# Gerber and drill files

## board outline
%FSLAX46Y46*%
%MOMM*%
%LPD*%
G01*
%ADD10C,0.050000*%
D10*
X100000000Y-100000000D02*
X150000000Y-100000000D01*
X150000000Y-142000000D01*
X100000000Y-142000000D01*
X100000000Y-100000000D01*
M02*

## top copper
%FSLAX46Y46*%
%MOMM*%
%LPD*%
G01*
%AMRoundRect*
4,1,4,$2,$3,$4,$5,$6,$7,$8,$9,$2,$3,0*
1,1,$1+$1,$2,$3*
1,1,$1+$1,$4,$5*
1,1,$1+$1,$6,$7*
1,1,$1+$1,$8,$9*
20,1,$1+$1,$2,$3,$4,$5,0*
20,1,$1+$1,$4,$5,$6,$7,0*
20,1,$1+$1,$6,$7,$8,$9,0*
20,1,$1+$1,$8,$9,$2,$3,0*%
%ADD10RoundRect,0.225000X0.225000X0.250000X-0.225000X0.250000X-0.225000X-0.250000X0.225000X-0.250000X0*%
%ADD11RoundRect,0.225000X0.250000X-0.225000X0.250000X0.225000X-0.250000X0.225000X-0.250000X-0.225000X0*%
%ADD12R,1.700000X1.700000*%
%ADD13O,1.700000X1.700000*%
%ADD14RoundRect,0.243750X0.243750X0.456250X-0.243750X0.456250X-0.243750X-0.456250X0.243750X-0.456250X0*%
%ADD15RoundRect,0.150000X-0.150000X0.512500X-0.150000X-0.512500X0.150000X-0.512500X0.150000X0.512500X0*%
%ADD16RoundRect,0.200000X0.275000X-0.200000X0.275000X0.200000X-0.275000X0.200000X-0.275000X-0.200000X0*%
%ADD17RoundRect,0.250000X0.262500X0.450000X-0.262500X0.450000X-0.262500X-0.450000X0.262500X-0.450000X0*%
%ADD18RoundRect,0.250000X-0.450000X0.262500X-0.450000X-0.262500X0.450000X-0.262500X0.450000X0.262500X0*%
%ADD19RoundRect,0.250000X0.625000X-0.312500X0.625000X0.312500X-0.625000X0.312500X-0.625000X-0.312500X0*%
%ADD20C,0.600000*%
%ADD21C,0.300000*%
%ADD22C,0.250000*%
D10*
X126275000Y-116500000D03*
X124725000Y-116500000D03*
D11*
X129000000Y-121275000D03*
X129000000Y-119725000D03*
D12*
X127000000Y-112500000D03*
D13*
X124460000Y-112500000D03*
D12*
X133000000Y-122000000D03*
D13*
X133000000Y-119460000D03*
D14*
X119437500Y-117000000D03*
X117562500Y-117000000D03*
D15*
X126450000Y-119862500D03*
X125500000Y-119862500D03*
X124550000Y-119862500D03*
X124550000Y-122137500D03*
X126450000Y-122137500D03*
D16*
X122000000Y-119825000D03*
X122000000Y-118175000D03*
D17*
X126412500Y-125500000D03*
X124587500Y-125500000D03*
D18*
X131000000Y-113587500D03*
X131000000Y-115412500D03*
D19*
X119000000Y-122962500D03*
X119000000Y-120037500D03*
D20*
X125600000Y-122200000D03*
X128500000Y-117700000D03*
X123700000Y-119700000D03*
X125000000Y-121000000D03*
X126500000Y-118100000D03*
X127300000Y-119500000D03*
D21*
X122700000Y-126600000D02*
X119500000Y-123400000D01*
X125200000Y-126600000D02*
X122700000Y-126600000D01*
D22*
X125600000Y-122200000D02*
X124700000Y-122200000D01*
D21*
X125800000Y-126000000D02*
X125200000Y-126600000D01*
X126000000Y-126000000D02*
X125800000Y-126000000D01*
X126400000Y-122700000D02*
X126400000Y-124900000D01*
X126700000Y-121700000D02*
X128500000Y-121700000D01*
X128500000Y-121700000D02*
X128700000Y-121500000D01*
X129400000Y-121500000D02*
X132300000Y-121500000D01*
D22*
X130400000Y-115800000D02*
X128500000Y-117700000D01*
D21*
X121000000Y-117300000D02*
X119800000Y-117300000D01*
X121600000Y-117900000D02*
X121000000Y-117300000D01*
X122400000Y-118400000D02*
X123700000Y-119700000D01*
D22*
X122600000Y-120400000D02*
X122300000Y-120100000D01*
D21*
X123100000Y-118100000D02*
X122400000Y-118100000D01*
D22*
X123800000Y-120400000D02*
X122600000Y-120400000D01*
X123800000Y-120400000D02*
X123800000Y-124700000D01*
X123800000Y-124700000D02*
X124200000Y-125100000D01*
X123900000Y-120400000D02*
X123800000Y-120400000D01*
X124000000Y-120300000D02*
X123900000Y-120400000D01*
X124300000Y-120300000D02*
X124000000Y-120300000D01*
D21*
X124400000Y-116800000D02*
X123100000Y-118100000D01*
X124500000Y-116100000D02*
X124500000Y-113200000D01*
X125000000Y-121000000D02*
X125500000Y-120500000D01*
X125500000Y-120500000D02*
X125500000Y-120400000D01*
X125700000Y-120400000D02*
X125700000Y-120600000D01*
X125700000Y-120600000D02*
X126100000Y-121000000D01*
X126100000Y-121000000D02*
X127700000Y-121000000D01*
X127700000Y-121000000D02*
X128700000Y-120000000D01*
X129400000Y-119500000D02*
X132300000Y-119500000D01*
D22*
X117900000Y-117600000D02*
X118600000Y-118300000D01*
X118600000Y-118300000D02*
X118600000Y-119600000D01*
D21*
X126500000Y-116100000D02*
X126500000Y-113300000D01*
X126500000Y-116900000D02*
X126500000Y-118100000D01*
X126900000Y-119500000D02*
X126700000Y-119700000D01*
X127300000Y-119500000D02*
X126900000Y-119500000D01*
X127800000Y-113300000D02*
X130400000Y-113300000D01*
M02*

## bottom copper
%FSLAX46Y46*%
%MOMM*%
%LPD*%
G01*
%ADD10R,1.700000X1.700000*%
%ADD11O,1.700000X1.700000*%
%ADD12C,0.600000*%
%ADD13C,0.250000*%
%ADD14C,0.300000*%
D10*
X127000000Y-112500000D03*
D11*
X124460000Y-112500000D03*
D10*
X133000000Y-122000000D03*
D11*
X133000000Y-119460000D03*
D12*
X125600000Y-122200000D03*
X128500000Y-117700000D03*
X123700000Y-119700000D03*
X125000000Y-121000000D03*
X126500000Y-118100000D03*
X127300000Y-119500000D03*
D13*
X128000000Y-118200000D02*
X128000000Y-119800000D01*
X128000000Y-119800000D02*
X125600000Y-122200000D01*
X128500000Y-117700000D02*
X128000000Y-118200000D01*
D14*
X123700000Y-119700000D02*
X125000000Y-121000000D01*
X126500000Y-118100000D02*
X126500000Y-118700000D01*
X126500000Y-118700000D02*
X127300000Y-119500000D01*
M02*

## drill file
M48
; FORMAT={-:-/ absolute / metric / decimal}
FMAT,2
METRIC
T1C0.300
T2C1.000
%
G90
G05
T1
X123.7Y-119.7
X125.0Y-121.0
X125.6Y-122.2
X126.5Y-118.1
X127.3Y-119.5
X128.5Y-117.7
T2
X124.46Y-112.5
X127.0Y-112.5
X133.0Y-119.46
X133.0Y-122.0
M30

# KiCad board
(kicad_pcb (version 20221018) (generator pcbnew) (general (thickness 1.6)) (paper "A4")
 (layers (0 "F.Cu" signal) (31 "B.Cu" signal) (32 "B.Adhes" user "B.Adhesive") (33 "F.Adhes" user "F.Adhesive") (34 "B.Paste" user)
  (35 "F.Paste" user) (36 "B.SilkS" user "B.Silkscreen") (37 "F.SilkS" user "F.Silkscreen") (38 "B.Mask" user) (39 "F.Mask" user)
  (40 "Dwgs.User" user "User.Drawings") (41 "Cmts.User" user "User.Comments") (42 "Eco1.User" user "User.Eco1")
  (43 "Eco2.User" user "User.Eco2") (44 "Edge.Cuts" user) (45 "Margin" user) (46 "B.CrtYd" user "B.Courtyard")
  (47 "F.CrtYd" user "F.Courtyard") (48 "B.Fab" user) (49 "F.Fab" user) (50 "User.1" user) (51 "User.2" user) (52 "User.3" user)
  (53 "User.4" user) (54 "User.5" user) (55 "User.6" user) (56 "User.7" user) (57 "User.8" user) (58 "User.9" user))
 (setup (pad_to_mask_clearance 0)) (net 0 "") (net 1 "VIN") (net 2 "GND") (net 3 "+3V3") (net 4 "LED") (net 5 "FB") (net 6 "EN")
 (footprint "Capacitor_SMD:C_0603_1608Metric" (layer "F.Cu") (at 125.5 116.5 180)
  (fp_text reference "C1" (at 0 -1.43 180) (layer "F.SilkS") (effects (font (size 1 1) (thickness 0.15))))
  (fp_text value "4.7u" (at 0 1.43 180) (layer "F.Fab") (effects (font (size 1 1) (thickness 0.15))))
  (pad "1" smd roundrect (at -0.775 0 180) (size 0.9 0.95) (layers "F.Cu" "F.Paste" "F.Mask") (roundrect_rratio 0.25) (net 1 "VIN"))
  (pad "2" smd roundrect (at 0.775 0 180) (size 0.9 0.95) (layers "F.Cu" "F.Paste" "F.Mask") (roundrect_rratio 0.25) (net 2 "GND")))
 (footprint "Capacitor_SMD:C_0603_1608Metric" (layer "F.Cu") (at 129 120.5 90)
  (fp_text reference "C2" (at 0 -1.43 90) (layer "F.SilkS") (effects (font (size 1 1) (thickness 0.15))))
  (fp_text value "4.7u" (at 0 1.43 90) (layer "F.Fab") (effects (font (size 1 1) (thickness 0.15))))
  (pad "1" smd roundrect (at -0.775 0 90) (size 0.9 0.95) (layers "F.Cu" "F.Paste" "F.Mask") (roundrect_rratio 0.25) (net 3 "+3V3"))
  (pad "2" smd roundrect (at 0.775 0 90) (size 0.9 0.95) (layers "F.Cu" "F.Paste" "F.Mask") (roundrect_rratio 0.25) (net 2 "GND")))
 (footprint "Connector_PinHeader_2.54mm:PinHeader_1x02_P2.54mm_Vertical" (layer "F.Cu") (at 127 112.5 -90)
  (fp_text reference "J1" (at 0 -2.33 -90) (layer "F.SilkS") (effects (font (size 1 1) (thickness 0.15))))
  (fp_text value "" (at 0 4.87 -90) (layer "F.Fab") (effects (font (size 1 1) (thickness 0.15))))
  (pad "1" thru_hole rect (at 0 0 270) (size 1.7 1.7) (drill 1) (layers "*.Cu" "*.Mask") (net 1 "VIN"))
  (pad "2" thru_hole oval (at 0 2.54 270) (size 1.7 1.7) (drill 1) (layers "*.Cu" "*.Mask") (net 2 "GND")))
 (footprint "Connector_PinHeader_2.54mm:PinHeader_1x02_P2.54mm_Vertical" (layer "F.Cu") (at 133 122 180)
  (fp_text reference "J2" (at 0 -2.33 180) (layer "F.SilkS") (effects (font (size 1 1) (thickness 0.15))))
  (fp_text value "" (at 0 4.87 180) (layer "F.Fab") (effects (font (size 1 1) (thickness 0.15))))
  (pad "1" thru_hole rect (at 0 0 180) (size 1.7 1.7) (drill 1) (layers "*.Cu" "*.Mask") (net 3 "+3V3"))
  (pad "2" thru_hole oval (at 0 2.54 180) (size 1.7 1.7) (drill 1) (layers "*.Cu" "*.Mask") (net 2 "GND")))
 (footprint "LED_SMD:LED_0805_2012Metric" (layer "F.Cu") (at 118.5 117 180)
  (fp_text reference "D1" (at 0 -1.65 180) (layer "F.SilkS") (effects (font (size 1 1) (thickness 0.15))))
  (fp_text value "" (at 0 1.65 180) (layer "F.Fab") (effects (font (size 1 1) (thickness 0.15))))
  (pad "1" smd roundrect (at -0.9375 0 180) (size 0.975 1.4) (layers "F.Cu" "F.Paste" "F.Mask") (roundrect_rratio 0.25) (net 2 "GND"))
  (pad "2" smd roundrect (at 0.9375 0 180) (size 0.975 1.4) (layers "F.Cu" "F.Paste" "F.Mask") (roundrect_rratio 0.25) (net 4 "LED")))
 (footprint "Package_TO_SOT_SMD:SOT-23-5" (layer "F.Cu") (at 125.5 121 -90)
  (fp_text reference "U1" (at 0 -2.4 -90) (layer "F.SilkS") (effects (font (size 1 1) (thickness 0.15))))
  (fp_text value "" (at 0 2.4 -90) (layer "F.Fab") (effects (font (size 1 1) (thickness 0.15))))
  (pad "1" smd roundrect (at -1.1375 -0.95 270) (size 1.325 0.6) (layers "F.Cu" "F.Paste" "F.Mask") (roundrect_rratio 0.25) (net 1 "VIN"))
  (pad "2" smd roundrect (at -1.1375 0 270) (size 1.325 0.6) (layers "F.Cu" "F.Paste" "F.Mask") (roundrect_rratio 0.25) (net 2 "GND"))
  (pad "3" smd roundrect (at -1.1375 0.95 270) (size 1.325 0.6) (layers "F.Cu" "F.Paste" "F.Mask") (roundrect_rratio 0.25) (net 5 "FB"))
  (pad "4" smd roundrect (at 1.1375 0.95 270) (size 1.325 0.6) (layers "F.Cu" "F.Paste" "F.Mask") (roundrect_rratio 0.25) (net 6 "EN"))
  (pad "5" smd roundrect (at 1.1375 -0.95 270) (size 1.325 0.6) (layers "F.Cu" "F.Paste" "F.Mask") (roundrect_rratio 0.25) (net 3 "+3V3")))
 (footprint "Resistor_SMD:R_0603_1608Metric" (layer "F.Cu") (at 122 119 90)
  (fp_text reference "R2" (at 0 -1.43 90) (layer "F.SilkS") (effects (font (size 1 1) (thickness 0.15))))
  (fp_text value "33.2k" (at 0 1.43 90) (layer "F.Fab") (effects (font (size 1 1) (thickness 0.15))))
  (pad "1" smd roundrect (at -0.825 0 90) (size 0.8 0.95) (layers "F.Cu" "F.Paste" "F.Mask") (roundrect_rratio 0.25) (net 5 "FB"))
  (pad "2" smd roundrect (at 0.825 0 90) (size 0.8 0.95) (layers "F.Cu" "F.Paste" "F.Mask") (roundrect_rratio 0.25) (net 2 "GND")))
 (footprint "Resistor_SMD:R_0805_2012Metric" (layer "F.Cu") (at 125.5 125.5 180)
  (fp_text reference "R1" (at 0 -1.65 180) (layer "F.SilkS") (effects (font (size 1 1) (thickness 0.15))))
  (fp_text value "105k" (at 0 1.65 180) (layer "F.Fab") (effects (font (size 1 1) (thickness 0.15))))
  (pad "1" smd roundrect (at -0.9125 0 180) (size 1.025 1.4) (layers "F.Cu" "F.Paste" "F.Mask") (roundrect_rratio 0.243902) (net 3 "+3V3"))
  (pad "2" smd roundrect (at 0.9125 0 180) (size 1.025 1.4) (layers "F.Cu" "F.Paste" "F.Mask") (roundrect_rratio 0.243902) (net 5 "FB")))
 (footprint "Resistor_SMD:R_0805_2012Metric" (layer "F.Cu") (at 131 114.5 -90)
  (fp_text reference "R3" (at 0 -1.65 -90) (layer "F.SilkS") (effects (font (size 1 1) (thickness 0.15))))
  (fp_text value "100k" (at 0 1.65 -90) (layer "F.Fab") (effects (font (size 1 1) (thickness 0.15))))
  (pad "1" smd roundrect (at -0.9125 0 270) (size 1.025 1.4) (layers "F.Cu" "F.Paste" "F.Mask") (roundrect_rratio 0.243902) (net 1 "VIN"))
  (pad "2" smd roundrect (at 0.9125 0 270) (size 1.025 1.4) (layers "F.Cu" "F.Paste" "F.Mask") (roundrect_rratio 0.243902) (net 6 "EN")))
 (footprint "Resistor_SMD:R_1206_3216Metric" (layer "F.Cu") (at 119 121.5 90)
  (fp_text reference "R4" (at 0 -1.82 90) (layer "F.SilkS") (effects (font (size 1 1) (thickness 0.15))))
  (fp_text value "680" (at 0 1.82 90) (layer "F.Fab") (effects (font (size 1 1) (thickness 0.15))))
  (pad "1" smd roundrect (at -1.4625 0 90) (size 1.125 1.75) (layers "F.Cu" "F.Paste" "F.Mask") (roundrect_rratio 0.222222) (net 3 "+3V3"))
  (pad "2" smd roundrect (at 1.4625 0 90) (size 1.125 1.75) (layers "F.Cu" "F.Paste" "F.Mask") (roundrect_rratio 0.222222) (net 4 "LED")))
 (gr_rect (start 100 100) (end 150 142) (stroke (width 0.05) (type default)) (fill none) (layer "Edge.Cuts"))
 (segment (start 122.7 126.6) (end 119.5 123.4) (width 0.3) (layer "F.Cu") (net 3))
 (segment (start 125.2 126.6) (end 122.7 126.6) (width 0.3) (layer "F.Cu") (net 3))
 (segment (start 125.6 122.2) (end 124.7 122.2) (width 0.25) (layer "F.Cu") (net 6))
 (segment (start 125.8 126) (end 125.2 126.6) (width 0.3) (layer "F.Cu") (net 3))
 (segment (start 126 126) (end 125.8 126) (width 0.3) (layer "F.Cu") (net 3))
 (segment (start 126.4 122.7) (end 126.4 124.9) (width 0.3) (layer "F.Cu") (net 3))
 (segment (start 126.7 121.7) (end 128.5 121.7) (width 0.3) (layer "F.Cu") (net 3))
 (segment (start 128.5 121.7) (end 128.7 121.5) (width 0.3) (layer "F.Cu") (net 3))
 (segment (start 129.4 121.5) (end 132.3 121.5) (width 0.3) (layer "F.Cu") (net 3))
 (segment (start 130.4 115.8) (end 128.5 117.7) (width 0.25) (layer "F.Cu") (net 6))
 (via (at 125.6 122.2) (size 0.6) (drill 0.3) (layers "F.Cu" "B.Cu") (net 6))
 (via (at 128.5 117.7) (size 0.6) (drill 0.3) (layers "F.Cu" "B.Cu") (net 6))
 (segment (start 121 117.3) (end 119.8 117.3) (width 0.3) (layer "F.Cu") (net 2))
 (segment (start 121.6 117.9) (end 121 117.3) (width 0.3) (layer "F.Cu") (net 2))
 (segment (start 122.4 118.4) (end 123.7 119.7) (width 0.3) (layer "F.Cu") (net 2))
 (segment (start 122.6 120.4) (end 122.3 120.1) (width 0.25) (layer "F.Cu") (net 5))
 (segment (start 123.1 118.1) (end 122.4 118.1) (width 0.3) (layer "F.Cu") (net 2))
 (segment (start 123.8 120.4) (end 122.6 120.4) (width 0.25) (layer "F.Cu") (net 5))
 (segment (start 123.8 120.4) (end 123.8 124.7) (width 0.25) (layer "F.Cu") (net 5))
 (segment (start 123.8 124.7) (end 124.2 125.1) (width 0.25) (layer "F.Cu") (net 5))
 (segment (start 123.9 120.4) (end 123.8 120.4) (width 0.25) (layer "F.Cu") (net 5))
 (segment (start 124 120.3) (end 123.9 120.4) (width 0.25) (layer "F.Cu") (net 5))
 (segment (start 124.3 120.3) (end 124 120.3) (width 0.25) (layer "F.Cu") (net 5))
 (segment (start 124.4 116.8) (end 123.1 118.1) (width 0.3) (layer "F.Cu") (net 2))
 (segment (start 124.5 116.1) (end 124.5 113.2) (width 0.3) (layer "F.Cu") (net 2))
 (segment (start 125 121) (end 125.5 120.5) (width 0.3) (layer "F.Cu") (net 2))
 (segment (start 125.5 120.5) (end 125.5 120.4) (width 0.3) (layer "F.Cu") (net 2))
 (segment (start 125.7 120.4) (end 125.7 120.6) (width 0.3) (layer "F.Cu") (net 2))
 (segment (start 125.7 120.6) (end 126.1 121) (width 0.3) (layer "F.Cu") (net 2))
 (segment (start 126.1 121) (end 127.7 121) (width 0.3) (layer "F.Cu") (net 2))
 (segment (start 127.7 121) (end 128.7 120) (width 0.3) (layer "F.Cu") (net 2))
 (segment (start 128 118.2) (end 128 119.8) (width 0.25) (layer "B.Cu") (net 6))
 (segment (start 128 119.8) (end 125.6 122.2) (width 0.25) (layer "B.Cu") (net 6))
 (segment (start 128.5 117.7) (end 128 118.2) (width 0.25) (layer "B.Cu") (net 6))
 (segment (start 129.4 119.5) (end 132.3 119.5) (width 0.3) (layer "F.Cu") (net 2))
 (via (at 123.7 119.7) (size 0.6) (drill 0.3) (layers "F.Cu" "B.Cu") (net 2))
 (via (at 125 121) (size 0.6) (drill 0.3) (layers "F.Cu" "B.Cu") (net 2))
 (segment (start 117.9 117.6) (end 118.6 118.3) (width 0.25) (layer "F.Cu") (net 4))
 (segment (start 118.6 118.3) (end 118.6 119.6) (width 0.25) (layer "F.Cu") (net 4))
 (segment (start 123.7 119.7) (end 125 121) (width 0.3) (layer "B.Cu") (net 2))
 (segment (start 126.5 116.1) (end 126.5 113.3) (width 0.3) (layer "F.Cu") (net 1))
 (segment (start 126.5 116.9) (end 126.5 118.1) (width 0.3) (layer "F.Cu") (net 1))
 (segment (start 126.9 119.5) (end 126.7 119.7) (width 0.3) (layer "F.Cu") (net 1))
 (segment (start 127.3 119.5) (end 126.9 119.5) (width 0.3) (layer "F.Cu") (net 1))
 (segment (start 127.8 113.3) (end 130.4 113.3) (width 0.3) (layer "F.Cu") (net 1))
 (via (at 126.5 118.1) (size 0.6) (drill 0.3) (layers "F.Cu" "B.Cu") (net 1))
 (via (at 127.3 119.5) (size 0.6) (drill 0.3) (layers "F.Cu" "B.Cu") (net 1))
 (segment (start 126.5 118.1) (end 126.5 118.7) (width 0.3) (layer "B.Cu") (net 1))
 (segment (start 126.5 118.7) (end 127.3 119.5) (width 0.3) (layer "B.Cu") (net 1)))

